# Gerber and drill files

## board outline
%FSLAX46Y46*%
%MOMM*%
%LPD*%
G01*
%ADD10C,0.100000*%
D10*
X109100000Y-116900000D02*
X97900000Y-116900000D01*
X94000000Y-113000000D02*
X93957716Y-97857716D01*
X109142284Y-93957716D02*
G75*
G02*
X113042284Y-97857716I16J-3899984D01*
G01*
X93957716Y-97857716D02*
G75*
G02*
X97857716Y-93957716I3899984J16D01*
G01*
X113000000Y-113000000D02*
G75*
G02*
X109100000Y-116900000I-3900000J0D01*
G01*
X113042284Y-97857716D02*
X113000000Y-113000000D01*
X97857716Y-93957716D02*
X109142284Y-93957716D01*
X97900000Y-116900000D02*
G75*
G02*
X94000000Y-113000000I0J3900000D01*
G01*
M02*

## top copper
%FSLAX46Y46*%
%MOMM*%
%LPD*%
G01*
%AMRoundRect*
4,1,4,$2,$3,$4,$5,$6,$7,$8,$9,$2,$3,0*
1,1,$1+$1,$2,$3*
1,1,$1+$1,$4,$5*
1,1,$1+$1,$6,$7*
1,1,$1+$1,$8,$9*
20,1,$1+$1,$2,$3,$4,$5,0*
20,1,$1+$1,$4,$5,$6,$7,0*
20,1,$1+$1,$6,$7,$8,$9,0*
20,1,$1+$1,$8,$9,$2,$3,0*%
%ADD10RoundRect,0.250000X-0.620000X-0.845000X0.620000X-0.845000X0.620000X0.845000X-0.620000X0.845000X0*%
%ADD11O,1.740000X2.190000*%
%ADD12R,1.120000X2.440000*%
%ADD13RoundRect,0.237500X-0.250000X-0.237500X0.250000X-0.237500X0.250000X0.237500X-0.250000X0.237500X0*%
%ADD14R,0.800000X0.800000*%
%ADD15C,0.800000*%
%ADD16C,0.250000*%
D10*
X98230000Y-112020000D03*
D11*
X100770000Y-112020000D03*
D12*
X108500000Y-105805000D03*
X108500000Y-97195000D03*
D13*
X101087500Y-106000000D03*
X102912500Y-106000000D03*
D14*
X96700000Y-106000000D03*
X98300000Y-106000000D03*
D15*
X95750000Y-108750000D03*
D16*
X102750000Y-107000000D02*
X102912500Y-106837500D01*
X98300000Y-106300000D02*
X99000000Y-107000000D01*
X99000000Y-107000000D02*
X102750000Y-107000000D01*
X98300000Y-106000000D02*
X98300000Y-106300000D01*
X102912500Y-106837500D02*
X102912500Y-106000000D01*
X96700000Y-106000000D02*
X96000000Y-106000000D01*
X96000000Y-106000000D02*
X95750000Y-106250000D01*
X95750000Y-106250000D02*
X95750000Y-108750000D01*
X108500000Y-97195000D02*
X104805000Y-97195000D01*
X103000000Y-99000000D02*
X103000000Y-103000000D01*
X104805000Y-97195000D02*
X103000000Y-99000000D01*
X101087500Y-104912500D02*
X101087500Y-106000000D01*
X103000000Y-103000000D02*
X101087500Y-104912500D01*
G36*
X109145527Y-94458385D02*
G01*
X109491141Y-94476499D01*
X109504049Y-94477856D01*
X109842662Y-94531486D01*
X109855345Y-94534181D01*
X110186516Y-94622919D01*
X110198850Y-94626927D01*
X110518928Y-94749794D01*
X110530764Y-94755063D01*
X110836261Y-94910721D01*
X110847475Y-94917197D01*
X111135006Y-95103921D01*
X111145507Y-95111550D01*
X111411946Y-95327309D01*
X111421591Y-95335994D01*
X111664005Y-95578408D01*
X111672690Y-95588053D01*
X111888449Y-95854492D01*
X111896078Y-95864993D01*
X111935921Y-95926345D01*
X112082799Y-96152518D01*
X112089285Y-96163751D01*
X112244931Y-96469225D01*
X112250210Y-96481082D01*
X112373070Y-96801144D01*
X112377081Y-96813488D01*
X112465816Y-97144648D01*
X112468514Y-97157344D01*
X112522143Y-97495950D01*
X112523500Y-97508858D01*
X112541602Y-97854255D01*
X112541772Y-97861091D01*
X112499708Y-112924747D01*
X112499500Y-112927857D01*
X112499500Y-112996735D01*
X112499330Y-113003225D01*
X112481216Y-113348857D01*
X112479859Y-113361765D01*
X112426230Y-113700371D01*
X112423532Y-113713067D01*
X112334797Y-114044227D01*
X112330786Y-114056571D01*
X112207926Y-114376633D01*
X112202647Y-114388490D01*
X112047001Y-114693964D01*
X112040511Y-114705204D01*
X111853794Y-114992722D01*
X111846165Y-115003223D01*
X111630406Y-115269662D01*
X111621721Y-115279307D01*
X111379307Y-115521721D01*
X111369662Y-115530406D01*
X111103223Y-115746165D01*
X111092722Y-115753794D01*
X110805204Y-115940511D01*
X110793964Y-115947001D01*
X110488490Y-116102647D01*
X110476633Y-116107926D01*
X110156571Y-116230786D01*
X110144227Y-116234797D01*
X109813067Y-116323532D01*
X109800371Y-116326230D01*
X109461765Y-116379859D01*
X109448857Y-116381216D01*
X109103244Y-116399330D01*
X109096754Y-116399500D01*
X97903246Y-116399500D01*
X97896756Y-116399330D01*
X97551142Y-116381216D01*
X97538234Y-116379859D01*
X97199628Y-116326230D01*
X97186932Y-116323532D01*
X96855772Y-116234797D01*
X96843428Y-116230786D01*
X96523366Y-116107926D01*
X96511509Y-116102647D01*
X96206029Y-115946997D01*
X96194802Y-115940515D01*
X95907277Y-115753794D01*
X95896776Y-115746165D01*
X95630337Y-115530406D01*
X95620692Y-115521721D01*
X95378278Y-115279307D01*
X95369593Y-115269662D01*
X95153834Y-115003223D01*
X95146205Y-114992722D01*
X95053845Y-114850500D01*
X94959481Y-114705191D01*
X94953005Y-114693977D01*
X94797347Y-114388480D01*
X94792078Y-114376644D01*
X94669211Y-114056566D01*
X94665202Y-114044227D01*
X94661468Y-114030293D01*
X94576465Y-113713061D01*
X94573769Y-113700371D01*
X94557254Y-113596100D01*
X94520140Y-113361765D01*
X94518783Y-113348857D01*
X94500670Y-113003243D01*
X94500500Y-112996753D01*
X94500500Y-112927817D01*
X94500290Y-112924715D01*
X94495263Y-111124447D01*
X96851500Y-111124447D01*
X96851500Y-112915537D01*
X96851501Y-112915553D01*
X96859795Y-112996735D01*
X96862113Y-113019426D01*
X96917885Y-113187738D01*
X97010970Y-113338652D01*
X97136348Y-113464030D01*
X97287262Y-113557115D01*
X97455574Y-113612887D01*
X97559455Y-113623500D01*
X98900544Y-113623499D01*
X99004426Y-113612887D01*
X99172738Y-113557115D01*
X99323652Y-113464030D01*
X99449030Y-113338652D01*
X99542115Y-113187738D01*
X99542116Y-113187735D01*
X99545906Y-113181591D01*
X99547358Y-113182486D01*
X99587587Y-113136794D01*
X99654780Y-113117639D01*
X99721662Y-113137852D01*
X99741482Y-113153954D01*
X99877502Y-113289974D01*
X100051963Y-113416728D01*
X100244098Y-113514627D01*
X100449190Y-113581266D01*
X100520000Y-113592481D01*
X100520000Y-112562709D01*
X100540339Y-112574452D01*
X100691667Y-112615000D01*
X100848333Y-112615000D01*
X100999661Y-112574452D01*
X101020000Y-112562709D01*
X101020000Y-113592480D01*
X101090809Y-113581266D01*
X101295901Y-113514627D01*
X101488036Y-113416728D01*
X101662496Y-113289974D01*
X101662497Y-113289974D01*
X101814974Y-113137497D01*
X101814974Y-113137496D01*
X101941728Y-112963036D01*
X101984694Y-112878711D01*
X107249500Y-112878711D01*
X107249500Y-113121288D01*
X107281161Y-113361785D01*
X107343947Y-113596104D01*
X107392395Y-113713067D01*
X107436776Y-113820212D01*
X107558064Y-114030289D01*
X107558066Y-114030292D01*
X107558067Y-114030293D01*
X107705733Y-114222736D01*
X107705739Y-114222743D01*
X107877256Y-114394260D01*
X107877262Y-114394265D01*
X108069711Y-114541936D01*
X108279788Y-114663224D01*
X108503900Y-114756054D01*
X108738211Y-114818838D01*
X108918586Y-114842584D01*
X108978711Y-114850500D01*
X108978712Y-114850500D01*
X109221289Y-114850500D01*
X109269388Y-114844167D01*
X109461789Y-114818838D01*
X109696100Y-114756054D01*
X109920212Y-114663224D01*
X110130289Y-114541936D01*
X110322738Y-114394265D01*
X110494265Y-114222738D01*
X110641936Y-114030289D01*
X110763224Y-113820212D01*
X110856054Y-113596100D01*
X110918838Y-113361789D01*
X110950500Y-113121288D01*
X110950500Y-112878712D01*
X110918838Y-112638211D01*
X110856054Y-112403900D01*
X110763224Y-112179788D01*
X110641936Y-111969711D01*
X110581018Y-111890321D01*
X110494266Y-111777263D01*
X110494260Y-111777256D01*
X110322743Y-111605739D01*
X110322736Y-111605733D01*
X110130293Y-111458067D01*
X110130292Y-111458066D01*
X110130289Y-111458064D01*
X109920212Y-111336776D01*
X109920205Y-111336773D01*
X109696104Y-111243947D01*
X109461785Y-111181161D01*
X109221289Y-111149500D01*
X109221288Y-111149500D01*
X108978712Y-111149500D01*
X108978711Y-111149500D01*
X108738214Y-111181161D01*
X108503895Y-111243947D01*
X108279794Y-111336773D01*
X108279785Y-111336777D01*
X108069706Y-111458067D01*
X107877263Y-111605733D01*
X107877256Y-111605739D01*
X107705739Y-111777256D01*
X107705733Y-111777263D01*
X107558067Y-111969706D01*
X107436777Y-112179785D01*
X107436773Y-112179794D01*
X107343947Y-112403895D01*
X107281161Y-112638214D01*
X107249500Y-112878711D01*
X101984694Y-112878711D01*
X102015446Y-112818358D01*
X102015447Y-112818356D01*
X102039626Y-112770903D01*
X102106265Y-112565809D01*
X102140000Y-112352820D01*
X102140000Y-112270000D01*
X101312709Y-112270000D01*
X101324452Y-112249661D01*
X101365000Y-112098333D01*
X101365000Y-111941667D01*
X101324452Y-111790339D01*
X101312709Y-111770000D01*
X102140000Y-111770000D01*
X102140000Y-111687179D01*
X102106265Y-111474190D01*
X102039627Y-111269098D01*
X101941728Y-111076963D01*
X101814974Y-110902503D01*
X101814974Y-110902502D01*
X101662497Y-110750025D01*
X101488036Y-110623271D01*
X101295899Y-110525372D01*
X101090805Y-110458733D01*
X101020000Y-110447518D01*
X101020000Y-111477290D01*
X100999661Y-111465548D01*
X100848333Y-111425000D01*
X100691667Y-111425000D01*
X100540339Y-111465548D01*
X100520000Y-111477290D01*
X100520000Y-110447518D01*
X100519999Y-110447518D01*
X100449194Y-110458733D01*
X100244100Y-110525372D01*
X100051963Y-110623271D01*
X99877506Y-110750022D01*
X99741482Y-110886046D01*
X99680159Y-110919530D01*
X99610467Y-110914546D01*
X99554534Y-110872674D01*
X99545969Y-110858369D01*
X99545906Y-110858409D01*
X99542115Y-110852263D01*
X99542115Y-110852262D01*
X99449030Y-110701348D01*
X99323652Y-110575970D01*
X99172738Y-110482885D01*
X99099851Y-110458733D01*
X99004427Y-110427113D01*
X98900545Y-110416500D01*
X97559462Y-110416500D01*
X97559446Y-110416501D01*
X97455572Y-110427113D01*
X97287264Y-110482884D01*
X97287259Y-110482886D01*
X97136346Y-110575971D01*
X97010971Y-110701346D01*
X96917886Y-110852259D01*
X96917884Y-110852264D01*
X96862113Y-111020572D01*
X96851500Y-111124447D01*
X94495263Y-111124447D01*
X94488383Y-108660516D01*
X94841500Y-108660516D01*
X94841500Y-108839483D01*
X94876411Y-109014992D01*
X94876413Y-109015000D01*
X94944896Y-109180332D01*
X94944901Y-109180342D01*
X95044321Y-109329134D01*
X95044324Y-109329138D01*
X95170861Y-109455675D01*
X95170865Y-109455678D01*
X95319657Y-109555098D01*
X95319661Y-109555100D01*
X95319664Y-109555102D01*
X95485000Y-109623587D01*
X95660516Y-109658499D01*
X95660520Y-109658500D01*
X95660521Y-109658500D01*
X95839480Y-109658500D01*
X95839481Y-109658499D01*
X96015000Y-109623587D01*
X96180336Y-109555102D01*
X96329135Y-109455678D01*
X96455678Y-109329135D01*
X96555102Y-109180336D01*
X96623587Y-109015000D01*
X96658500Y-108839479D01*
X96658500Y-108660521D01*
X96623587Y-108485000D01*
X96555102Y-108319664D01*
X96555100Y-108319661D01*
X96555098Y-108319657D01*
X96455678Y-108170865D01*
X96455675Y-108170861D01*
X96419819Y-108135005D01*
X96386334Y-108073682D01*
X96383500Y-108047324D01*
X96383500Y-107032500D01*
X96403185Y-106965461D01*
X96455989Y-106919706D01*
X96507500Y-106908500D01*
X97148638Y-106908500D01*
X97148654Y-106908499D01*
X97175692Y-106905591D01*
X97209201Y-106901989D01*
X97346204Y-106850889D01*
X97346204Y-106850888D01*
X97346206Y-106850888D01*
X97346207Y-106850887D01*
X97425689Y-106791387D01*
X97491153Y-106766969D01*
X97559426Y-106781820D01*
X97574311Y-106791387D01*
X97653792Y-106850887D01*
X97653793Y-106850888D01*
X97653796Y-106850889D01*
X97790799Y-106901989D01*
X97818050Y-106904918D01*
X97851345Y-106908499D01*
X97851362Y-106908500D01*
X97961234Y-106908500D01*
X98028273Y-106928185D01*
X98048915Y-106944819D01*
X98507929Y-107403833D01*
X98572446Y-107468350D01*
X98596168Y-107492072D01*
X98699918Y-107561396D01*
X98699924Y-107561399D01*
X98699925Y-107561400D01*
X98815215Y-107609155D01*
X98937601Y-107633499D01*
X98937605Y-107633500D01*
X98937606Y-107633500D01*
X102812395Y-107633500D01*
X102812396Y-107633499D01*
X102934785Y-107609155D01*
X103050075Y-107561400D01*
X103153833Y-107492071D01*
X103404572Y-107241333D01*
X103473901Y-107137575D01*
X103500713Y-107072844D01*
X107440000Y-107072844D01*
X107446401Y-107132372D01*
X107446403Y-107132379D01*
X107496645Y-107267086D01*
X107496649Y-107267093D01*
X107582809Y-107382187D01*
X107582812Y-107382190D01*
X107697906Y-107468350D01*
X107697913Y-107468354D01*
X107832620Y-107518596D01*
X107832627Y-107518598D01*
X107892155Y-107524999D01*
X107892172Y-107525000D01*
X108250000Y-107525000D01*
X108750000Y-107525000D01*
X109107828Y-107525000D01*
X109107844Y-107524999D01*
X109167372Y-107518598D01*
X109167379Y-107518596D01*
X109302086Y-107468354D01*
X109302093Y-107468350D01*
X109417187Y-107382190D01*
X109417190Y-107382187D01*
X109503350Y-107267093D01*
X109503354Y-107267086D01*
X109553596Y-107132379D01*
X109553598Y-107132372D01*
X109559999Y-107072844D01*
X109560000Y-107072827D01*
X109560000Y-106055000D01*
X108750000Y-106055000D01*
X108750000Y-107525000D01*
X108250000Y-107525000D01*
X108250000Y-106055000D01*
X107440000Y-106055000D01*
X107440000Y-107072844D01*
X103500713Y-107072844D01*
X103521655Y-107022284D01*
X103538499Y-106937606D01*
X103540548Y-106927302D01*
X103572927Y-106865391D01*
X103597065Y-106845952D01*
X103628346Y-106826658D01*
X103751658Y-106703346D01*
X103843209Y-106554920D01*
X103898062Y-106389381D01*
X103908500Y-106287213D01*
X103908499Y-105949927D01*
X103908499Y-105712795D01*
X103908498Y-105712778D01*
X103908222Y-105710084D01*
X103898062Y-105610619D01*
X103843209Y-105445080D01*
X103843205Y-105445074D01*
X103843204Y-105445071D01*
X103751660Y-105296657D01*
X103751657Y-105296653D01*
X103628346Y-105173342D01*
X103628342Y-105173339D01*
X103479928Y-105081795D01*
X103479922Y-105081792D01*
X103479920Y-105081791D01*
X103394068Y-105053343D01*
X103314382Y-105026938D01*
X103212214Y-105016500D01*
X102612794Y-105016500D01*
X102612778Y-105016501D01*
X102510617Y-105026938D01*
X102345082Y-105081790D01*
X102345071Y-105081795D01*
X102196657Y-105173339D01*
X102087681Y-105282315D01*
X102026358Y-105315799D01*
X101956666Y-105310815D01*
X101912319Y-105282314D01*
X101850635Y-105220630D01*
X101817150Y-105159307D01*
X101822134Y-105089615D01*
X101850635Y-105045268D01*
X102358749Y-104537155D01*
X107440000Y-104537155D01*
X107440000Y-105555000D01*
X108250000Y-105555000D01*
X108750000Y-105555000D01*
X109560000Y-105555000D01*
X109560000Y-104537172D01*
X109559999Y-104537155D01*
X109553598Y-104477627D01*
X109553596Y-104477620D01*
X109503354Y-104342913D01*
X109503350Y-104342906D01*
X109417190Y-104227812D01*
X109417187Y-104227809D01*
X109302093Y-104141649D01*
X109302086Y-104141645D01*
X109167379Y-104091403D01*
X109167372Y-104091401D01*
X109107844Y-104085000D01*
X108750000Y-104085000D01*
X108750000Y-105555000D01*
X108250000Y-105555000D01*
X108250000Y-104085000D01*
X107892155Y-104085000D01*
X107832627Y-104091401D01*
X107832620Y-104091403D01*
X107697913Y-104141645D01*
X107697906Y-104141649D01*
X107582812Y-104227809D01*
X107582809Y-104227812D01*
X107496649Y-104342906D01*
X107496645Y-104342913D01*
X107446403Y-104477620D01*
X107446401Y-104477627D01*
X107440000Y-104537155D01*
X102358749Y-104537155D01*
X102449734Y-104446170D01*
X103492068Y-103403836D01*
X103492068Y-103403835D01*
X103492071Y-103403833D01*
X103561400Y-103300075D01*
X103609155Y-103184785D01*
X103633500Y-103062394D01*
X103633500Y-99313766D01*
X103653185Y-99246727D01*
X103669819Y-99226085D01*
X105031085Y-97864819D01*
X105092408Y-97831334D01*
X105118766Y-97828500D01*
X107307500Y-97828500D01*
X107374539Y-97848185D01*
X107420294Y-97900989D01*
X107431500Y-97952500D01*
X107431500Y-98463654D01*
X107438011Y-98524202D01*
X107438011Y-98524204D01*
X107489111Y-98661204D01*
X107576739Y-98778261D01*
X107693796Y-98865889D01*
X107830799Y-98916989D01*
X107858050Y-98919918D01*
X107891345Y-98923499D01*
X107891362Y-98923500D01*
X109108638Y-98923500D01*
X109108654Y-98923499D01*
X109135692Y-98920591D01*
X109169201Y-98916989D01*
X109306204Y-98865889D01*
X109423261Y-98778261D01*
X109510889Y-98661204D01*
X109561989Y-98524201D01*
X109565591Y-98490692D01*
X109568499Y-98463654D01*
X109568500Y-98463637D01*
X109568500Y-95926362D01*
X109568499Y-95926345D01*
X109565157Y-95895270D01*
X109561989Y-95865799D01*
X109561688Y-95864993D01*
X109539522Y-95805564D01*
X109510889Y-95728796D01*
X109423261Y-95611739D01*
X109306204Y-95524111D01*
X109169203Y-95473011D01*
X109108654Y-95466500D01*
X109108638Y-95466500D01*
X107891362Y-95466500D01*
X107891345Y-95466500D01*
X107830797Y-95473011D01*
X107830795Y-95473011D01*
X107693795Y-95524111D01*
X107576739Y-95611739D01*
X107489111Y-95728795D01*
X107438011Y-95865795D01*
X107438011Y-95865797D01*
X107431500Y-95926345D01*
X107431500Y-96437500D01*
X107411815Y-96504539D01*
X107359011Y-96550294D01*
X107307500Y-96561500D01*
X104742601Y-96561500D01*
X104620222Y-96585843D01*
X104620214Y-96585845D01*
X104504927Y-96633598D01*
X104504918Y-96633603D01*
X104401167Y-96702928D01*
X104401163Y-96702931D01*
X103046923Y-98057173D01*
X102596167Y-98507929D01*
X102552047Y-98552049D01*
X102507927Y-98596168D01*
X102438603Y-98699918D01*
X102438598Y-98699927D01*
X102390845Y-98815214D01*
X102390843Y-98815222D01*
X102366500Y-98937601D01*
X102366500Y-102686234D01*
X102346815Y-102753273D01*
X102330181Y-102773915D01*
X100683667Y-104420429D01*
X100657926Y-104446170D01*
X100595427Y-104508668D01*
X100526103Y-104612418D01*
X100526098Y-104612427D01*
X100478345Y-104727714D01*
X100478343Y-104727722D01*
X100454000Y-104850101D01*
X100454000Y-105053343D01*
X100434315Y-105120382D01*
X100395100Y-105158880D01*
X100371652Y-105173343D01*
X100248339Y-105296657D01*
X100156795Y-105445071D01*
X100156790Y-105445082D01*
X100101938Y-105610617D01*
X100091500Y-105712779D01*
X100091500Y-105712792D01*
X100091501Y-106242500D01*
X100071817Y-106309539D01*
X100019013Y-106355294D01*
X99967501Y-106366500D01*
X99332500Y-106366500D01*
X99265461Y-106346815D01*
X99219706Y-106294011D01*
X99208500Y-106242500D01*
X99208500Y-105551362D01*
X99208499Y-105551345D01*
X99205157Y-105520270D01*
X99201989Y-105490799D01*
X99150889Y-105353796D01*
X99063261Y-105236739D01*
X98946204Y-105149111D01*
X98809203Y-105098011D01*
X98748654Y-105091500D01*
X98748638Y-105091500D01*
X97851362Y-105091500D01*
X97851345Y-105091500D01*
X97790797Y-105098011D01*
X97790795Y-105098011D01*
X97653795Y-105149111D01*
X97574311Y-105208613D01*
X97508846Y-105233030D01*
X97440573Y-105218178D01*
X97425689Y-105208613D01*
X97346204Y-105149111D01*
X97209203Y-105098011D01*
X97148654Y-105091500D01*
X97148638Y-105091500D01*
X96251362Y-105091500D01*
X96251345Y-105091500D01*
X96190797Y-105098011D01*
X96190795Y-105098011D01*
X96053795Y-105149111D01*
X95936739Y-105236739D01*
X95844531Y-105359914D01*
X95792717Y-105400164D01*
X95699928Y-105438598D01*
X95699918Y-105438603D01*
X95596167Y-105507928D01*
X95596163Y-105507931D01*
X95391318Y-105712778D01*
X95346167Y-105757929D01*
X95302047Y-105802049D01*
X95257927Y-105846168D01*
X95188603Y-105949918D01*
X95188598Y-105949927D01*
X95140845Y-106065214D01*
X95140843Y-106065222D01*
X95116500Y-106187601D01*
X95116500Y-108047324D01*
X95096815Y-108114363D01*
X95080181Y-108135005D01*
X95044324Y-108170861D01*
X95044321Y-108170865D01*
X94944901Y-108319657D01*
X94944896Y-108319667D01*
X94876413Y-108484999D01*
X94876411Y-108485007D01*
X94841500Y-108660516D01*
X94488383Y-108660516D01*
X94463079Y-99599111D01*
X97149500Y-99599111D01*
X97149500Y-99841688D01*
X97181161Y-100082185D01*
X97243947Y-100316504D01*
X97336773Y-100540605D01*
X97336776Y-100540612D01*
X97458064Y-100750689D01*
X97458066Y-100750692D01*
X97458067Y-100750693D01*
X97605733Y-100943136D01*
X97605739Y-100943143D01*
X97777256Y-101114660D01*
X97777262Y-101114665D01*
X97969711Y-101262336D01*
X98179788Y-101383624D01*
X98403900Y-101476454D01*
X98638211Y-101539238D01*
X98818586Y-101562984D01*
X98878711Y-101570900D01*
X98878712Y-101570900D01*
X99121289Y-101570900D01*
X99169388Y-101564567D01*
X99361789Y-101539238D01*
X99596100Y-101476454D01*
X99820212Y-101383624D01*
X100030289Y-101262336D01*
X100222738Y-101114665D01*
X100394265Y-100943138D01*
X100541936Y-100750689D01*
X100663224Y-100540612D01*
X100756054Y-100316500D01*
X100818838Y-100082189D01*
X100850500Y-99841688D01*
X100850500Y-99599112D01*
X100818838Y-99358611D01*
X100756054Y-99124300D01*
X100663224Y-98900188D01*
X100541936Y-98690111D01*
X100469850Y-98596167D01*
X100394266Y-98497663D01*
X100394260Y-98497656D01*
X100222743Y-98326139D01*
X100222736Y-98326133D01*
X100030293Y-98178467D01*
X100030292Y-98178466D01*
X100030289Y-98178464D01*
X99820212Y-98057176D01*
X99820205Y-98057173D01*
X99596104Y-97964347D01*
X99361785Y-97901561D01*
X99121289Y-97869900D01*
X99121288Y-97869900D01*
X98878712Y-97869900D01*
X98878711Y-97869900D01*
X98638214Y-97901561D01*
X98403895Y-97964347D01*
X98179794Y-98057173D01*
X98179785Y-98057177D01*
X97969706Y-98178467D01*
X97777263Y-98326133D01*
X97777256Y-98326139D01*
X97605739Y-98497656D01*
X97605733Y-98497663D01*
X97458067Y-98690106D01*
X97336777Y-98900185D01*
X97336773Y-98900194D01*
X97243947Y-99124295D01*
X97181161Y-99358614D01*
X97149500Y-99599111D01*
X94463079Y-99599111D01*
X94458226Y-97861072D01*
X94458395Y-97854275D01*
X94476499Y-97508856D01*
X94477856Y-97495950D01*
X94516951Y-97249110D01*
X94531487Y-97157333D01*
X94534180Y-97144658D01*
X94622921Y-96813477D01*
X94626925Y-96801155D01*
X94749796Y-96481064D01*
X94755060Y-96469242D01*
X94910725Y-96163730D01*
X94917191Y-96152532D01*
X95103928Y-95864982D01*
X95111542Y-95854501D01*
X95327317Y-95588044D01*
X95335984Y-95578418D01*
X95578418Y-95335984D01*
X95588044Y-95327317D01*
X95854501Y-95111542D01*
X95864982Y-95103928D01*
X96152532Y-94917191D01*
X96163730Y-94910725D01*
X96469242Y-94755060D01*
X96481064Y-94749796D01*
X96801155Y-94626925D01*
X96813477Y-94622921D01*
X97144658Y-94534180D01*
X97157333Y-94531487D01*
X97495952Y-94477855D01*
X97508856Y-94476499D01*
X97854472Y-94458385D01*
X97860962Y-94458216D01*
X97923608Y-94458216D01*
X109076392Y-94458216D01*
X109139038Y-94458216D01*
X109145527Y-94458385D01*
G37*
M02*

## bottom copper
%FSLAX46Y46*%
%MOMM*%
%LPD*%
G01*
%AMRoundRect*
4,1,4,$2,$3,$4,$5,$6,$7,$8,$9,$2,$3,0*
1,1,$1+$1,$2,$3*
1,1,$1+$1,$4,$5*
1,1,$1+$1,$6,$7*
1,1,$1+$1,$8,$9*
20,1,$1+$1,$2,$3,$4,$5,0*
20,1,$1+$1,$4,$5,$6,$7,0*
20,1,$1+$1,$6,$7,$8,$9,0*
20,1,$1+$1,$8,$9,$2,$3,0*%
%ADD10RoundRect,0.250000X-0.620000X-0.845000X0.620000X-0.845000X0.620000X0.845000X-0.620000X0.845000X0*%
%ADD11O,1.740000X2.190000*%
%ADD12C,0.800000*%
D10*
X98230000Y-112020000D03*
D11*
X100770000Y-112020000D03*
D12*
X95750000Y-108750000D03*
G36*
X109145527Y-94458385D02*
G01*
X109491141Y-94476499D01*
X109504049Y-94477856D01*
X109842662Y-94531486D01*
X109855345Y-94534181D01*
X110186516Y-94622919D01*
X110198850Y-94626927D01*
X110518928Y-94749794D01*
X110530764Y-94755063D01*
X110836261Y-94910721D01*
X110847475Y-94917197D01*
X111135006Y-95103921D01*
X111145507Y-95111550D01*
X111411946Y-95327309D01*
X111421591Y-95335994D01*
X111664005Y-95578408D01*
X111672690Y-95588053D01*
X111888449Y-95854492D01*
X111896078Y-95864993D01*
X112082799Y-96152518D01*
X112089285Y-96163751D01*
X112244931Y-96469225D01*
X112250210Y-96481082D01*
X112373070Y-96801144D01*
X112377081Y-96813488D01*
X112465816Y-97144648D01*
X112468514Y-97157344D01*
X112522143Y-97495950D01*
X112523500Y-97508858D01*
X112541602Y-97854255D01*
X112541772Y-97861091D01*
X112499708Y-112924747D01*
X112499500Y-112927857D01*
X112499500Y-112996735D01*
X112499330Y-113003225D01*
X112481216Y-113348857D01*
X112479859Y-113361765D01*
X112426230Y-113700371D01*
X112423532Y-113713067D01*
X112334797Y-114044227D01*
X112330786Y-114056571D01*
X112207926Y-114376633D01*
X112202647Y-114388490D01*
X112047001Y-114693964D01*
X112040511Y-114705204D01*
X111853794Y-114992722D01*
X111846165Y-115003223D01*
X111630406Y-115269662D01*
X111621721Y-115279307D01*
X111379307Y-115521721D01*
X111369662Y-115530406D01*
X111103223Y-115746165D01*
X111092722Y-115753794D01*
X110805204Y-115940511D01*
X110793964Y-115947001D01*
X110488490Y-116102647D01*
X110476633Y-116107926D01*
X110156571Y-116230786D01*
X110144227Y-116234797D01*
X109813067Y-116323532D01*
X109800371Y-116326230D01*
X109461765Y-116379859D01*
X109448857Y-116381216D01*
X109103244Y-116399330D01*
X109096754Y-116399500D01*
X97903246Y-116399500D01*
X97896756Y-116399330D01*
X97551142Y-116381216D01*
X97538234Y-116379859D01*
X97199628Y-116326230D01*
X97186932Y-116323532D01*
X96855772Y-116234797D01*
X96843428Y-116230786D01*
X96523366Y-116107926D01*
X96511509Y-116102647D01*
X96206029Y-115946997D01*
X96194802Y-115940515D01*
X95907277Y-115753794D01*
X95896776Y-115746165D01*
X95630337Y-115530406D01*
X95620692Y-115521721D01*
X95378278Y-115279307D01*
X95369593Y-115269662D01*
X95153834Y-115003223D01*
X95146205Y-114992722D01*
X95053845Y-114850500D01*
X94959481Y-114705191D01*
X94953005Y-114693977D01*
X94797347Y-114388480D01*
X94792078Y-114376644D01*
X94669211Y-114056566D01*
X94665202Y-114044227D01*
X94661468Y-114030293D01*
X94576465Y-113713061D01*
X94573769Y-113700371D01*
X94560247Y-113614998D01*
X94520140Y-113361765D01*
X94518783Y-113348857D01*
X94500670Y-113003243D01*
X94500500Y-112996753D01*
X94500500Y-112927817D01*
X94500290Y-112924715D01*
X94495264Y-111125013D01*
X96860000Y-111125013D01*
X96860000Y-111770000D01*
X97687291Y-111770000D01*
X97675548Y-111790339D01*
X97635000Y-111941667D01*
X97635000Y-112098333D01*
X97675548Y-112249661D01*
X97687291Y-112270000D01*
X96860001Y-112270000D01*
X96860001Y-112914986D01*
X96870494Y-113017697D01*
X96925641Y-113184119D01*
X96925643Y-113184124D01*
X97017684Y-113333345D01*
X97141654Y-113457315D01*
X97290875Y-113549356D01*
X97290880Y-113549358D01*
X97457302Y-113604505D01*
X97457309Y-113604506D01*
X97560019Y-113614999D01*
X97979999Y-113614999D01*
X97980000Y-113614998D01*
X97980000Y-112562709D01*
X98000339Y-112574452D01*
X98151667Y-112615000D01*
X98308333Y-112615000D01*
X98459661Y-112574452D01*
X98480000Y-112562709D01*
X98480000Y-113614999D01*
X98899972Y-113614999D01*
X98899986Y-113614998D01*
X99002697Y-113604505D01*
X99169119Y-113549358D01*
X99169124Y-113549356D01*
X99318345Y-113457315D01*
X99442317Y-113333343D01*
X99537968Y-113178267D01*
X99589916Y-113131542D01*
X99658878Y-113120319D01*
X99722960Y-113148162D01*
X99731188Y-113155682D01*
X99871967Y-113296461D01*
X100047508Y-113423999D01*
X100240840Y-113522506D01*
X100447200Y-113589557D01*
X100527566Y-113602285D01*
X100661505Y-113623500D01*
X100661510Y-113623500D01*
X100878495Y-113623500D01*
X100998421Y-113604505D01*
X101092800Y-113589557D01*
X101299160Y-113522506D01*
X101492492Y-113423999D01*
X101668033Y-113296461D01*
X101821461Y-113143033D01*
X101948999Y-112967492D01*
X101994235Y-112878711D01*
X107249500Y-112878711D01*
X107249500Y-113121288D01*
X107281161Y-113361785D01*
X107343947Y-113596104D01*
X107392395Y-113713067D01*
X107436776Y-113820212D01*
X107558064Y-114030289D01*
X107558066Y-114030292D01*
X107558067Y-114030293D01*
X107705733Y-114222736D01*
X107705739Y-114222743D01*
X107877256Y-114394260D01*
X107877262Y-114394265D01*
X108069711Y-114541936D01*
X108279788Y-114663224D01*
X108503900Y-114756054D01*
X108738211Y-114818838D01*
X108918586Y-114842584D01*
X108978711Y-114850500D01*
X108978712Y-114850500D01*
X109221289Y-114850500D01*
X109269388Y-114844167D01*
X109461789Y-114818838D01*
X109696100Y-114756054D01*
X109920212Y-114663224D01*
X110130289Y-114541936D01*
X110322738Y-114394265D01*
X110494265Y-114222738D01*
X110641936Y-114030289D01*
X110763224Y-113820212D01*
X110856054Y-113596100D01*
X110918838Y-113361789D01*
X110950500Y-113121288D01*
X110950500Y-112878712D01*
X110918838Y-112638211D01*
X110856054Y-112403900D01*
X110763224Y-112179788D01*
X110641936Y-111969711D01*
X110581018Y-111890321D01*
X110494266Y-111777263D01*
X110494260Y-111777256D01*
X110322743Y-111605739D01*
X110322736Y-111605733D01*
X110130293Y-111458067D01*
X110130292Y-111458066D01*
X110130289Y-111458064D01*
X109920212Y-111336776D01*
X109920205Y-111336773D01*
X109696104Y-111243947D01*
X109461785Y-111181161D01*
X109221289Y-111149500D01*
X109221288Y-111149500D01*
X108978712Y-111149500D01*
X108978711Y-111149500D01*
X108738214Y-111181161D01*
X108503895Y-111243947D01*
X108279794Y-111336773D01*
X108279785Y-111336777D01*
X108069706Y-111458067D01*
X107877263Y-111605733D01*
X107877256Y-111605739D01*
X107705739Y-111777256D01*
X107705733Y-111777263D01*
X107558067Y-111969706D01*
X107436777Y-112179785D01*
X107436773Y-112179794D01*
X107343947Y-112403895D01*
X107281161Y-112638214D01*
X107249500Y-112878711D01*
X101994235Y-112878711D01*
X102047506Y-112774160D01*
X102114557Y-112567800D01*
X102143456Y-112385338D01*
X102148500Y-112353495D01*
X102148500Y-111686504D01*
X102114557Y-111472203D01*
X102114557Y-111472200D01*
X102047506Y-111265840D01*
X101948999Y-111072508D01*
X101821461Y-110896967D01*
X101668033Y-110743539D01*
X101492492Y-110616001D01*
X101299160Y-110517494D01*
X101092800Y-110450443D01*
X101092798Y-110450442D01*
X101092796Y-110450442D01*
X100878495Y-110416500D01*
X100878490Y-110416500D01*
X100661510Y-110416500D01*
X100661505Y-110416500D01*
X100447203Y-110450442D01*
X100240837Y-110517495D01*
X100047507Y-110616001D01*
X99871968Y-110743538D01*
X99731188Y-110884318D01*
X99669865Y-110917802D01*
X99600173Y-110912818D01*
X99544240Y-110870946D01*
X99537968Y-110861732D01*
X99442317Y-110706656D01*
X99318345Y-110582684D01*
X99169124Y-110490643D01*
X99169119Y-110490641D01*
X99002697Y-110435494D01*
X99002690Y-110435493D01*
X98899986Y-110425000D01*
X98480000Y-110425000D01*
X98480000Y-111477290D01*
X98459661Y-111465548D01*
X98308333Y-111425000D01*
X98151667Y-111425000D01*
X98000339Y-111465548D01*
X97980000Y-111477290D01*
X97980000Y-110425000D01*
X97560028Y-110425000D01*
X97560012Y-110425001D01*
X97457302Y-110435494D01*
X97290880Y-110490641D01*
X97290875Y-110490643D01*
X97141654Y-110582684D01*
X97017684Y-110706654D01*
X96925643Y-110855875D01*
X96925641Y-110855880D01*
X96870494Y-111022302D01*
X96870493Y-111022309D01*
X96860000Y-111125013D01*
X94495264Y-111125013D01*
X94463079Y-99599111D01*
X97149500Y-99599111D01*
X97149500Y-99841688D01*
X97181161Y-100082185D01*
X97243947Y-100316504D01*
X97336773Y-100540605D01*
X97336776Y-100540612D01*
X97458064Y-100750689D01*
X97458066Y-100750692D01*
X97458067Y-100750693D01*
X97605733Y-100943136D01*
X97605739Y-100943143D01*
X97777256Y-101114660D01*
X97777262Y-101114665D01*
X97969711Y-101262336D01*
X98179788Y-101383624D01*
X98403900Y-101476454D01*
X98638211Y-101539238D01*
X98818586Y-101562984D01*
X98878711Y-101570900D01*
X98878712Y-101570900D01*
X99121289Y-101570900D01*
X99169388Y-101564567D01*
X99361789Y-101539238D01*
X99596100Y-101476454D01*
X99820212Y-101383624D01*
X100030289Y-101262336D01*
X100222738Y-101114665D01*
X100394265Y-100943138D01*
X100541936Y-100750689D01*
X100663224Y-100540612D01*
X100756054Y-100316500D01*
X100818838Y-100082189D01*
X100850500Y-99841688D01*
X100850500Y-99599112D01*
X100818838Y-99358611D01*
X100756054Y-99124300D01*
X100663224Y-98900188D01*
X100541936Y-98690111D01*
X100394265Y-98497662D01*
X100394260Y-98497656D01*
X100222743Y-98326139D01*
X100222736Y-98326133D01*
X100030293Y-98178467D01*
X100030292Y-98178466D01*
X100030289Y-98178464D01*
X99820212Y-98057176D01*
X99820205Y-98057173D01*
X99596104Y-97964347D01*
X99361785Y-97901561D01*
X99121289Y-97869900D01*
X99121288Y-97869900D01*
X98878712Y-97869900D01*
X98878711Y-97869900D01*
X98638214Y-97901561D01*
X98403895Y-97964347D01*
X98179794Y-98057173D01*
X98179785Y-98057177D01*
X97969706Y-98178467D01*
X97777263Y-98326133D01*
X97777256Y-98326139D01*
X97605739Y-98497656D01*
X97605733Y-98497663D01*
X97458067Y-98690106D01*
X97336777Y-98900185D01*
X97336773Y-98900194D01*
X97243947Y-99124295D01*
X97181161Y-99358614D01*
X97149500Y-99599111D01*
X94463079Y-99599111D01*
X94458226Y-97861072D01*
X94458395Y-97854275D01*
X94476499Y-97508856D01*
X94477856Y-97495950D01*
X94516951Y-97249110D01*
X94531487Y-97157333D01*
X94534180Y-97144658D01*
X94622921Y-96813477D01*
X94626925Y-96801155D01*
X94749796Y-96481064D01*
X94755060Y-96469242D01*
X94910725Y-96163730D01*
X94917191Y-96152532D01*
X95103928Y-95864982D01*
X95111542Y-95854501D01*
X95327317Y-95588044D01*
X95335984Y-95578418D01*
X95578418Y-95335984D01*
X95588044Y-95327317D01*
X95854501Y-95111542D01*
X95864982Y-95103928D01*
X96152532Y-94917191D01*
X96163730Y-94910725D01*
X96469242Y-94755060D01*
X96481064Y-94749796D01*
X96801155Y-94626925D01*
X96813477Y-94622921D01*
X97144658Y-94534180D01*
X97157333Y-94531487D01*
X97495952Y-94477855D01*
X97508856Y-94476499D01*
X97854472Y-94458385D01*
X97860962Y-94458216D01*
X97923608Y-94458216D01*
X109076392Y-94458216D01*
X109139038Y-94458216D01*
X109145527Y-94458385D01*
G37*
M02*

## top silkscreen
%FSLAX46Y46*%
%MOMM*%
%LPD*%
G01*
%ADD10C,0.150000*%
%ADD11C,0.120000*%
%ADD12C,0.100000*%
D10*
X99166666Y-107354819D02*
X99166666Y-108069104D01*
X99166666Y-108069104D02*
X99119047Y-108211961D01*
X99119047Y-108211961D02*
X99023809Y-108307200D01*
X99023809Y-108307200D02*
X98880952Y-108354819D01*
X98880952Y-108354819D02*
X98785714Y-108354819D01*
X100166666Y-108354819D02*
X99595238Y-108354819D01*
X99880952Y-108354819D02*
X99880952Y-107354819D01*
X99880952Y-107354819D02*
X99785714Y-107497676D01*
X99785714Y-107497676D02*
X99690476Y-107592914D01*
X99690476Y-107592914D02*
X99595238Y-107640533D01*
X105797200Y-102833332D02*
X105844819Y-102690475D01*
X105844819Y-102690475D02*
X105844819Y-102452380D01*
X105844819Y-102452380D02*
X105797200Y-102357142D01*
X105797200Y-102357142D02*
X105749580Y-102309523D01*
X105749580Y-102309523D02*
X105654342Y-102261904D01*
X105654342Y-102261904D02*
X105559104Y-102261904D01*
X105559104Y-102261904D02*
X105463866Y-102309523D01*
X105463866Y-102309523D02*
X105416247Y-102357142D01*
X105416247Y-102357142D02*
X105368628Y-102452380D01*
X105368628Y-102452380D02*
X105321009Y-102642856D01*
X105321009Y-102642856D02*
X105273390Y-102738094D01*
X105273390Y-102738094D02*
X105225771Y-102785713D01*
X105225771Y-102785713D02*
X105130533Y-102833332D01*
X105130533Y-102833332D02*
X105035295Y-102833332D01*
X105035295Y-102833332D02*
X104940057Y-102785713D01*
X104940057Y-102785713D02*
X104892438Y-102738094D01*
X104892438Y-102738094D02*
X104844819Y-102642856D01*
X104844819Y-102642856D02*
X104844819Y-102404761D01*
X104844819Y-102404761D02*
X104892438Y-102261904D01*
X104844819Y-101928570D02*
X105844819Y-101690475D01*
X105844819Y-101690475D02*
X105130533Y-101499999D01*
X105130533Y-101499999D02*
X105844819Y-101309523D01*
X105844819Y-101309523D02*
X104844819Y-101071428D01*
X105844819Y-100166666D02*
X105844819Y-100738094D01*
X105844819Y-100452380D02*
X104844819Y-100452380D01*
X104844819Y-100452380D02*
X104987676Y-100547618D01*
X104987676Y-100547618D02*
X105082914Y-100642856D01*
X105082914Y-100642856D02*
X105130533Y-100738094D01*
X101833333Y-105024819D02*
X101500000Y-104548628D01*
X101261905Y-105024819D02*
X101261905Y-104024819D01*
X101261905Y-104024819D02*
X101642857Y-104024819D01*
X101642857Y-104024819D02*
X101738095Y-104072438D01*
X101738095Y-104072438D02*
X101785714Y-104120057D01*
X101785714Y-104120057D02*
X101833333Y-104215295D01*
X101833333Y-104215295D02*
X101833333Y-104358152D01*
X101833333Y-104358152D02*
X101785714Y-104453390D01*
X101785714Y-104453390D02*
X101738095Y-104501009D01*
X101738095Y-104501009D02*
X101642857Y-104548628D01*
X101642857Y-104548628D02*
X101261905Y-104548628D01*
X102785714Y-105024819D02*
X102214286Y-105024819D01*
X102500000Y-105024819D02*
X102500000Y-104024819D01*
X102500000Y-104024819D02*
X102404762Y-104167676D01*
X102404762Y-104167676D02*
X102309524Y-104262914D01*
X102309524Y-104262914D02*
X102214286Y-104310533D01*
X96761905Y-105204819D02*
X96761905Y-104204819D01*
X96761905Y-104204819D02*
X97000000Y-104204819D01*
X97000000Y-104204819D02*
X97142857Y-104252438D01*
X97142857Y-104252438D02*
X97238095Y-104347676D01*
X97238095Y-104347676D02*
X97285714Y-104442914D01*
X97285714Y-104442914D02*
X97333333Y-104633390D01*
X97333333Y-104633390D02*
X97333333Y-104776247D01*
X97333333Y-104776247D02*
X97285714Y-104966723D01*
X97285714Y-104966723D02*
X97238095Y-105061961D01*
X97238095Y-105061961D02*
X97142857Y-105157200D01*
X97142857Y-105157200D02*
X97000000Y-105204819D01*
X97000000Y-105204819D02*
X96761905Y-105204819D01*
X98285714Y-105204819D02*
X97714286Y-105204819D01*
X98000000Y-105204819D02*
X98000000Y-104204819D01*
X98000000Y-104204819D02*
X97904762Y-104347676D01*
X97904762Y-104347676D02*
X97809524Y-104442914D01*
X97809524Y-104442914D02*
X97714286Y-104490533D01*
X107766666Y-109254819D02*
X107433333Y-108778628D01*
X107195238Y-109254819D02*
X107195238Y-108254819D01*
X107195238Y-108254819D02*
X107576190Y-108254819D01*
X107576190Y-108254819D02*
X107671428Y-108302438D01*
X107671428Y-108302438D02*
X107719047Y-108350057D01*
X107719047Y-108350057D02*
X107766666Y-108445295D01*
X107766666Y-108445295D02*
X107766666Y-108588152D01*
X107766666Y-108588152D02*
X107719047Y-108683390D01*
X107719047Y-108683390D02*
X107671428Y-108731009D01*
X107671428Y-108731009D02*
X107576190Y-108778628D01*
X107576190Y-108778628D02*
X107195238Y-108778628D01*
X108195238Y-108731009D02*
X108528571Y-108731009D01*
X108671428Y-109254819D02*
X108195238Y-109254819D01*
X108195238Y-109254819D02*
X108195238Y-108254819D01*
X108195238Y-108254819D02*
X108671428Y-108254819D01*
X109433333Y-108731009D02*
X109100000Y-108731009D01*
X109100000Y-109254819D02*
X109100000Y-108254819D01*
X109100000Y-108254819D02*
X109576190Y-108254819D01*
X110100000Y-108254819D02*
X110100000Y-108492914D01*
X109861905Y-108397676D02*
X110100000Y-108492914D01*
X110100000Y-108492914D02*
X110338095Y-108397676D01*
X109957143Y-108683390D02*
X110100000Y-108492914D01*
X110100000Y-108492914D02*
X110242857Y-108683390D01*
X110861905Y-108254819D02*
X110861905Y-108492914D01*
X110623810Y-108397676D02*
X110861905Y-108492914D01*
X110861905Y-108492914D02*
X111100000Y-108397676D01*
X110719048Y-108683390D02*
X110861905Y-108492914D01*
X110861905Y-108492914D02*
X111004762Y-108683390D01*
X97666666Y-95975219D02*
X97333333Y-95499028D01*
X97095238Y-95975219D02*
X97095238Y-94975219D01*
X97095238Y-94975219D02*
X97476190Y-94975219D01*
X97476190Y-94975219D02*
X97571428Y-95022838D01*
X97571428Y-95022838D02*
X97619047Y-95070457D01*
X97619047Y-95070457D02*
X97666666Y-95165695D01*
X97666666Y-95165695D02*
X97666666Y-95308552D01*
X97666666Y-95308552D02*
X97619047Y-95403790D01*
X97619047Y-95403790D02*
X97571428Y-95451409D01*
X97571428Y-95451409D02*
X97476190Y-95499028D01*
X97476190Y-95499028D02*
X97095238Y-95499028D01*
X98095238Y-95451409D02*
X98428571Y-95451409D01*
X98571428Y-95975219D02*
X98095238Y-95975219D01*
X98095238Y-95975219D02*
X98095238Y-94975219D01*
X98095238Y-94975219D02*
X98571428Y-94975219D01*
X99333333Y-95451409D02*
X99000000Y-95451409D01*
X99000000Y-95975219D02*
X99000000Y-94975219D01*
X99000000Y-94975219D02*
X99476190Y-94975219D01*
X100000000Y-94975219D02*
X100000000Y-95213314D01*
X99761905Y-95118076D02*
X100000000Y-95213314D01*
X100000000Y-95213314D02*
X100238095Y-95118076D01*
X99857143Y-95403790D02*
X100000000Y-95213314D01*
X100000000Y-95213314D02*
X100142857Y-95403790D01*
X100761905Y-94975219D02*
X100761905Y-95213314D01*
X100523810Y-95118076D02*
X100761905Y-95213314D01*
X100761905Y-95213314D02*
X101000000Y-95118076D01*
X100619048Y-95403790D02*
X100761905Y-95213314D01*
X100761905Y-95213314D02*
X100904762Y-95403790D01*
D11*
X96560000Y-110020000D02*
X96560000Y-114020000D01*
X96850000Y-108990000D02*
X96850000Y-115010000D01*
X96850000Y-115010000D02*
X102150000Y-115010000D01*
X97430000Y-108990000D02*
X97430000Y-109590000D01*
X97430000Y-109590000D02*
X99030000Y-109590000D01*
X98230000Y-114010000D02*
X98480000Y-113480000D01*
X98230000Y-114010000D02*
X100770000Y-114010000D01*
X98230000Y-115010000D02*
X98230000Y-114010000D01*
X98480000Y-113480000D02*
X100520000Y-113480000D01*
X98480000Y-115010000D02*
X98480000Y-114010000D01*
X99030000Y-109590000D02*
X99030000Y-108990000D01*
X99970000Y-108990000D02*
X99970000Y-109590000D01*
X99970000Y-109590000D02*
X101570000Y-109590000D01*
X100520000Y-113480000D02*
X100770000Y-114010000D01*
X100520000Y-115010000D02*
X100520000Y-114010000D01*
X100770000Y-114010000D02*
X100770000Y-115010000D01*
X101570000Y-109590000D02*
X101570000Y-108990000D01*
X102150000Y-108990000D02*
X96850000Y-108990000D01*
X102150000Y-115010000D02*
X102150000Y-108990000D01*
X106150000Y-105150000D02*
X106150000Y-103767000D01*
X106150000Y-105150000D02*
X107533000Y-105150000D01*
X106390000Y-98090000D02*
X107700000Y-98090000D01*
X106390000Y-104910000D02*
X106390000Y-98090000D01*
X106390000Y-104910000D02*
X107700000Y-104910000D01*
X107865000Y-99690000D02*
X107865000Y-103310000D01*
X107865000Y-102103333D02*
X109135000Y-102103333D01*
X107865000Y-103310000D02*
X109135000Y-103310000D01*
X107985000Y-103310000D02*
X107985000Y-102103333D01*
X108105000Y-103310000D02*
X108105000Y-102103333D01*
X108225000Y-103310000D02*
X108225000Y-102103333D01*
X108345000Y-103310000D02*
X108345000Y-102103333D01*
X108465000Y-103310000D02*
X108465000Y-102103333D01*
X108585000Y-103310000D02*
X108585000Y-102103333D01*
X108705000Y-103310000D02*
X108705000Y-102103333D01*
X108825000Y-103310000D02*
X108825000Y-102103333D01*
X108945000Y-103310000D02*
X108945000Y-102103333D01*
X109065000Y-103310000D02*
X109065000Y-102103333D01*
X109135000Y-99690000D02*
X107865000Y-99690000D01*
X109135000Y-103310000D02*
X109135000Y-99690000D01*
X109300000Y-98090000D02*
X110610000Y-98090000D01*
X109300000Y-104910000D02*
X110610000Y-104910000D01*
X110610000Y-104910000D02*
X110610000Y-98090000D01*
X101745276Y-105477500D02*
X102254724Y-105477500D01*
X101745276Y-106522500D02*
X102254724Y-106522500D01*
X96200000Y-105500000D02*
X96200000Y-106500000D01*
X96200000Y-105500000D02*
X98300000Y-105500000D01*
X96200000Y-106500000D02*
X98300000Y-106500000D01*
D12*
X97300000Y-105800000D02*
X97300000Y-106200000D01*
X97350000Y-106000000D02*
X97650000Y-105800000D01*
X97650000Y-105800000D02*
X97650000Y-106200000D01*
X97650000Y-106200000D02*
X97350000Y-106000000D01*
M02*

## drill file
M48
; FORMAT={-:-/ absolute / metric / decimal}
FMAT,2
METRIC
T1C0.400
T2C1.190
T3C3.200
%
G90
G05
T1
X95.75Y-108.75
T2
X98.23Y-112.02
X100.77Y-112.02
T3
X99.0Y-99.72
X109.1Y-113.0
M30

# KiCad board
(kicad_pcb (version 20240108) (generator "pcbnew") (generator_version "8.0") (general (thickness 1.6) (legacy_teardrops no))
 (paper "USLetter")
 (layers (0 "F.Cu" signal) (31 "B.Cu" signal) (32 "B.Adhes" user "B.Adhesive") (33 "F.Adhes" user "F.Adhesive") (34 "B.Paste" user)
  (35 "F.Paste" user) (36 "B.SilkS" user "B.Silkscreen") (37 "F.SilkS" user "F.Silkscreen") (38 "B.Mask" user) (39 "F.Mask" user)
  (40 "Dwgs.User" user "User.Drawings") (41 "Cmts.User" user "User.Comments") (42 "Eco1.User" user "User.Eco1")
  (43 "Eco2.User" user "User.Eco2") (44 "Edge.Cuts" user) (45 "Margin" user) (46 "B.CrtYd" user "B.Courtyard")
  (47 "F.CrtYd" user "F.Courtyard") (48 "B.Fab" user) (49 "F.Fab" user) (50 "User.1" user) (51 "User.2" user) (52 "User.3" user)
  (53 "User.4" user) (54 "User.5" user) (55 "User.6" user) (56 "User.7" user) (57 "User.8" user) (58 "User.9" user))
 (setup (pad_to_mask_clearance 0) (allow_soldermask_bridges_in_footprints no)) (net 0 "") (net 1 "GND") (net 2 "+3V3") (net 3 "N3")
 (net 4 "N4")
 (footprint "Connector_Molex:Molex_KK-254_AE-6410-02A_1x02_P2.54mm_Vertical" (layer "F.Cu") (at 98.23 112.02)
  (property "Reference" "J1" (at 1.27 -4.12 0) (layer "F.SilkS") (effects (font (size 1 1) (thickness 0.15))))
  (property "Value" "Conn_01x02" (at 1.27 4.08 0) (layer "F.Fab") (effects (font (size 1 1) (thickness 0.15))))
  (fp_line (start -1.67 -2) (end -1.67 2) (stroke (width 0.12) (type solid)) (layer "F.SilkS"))
  (fp_line (start -1.38 -3.03) (end -1.38 2.99) (stroke (width 0.12) (type solid)) (layer "F.SilkS"))
  (fp_line (start -1.38 2.99) (end 3.92 2.99) (stroke (width 0.12) (type solid)) (layer "F.SilkS"))
  (fp_line (start -0.8 -3.03) (end -0.8 -2.43) (stroke (width 0.12) (type solid)) (layer "F.SilkS"))
  (fp_line (start -0.8 -2.43) (end 0.8 -2.43) (stroke (width 0.12) (type solid)) (layer "F.SilkS"))
  (fp_line (start 0 1.99) (end 0.25 1.46) (stroke (width 0.12) (type solid)) (layer "F.SilkS"))
  (fp_line (start 0 1.99) (end 2.54 1.99) (stroke (width 0.12) (type solid)) (layer "F.SilkS"))
  (fp_line (start 0 2.99) (end 0 1.99) (stroke (width 0.12) (type solid)) (layer "F.SilkS"))
  (fp_line (start 0.25 1.46) (end 2.29 1.46) (stroke (width 0.12) (type solid)) (layer "F.SilkS"))
  (fp_line (start 0.25 2.99) (end 0.25 1.99) (stroke (width 0.12) (type solid)) (layer "F.SilkS"))
  (fp_line (start 0.8 -2.43) (end 0.8 -3.03) (stroke (width 0.12) (type solid)) (layer "F.SilkS"))
  (fp_line (start 1.74 -3.03) (end 1.74 -2.43) (stroke (width 0.12) (type solid)) (layer "F.SilkS"))
  (fp_line (start 1.74 -2.43) (end 3.34 -2.43) (stroke (width 0.12) (type solid)) (layer "F.SilkS"))
  (fp_line (start 2.29 1.46) (end 2.54 1.99) (stroke (width 0.12) (type solid)) (layer "F.SilkS"))
  (fp_line (start 2.29 2.99) (end 2.29 1.99) (stroke (width 0.12) (type solid)) (layer "F.SilkS"))
  (fp_line (start 2.54 1.99) (end 2.54 2.99) (stroke (width 0.12) (type solid)) (layer "F.SilkS"))
  (fp_line (start 3.34 -2.43) (end 3.34 -3.03) (stroke (width 0.12) (type solid)) (layer "F.SilkS"))
  (fp_line (start 3.92 -3.03) (end -1.38 -3.03) (stroke (width 0.12) (type solid)) (layer "F.SilkS"))
  (fp_line (start 3.92 2.99) (end 3.92 -3.03) (stroke (width 0.12) (type solid)) (layer "F.SilkS"))
  (pad "1" thru_hole roundrect (at 0 0) (size 1.74 2.19) (drill 1.19) (layers "*.Cu" "*.Mask") (remove_unused_layers no)
   (roundrect_rratio 0.143678) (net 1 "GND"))
  (pad "2" thru_hole oval (at 2.54 0) (size 1.74 2.19) (drill 1.19) (layers "*.Cu" "*.Mask") (remove_unused_layers no) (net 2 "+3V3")))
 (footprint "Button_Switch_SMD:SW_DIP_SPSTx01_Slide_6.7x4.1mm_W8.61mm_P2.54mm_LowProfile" (layer "F.Cu") (at 108.5 101.5 90)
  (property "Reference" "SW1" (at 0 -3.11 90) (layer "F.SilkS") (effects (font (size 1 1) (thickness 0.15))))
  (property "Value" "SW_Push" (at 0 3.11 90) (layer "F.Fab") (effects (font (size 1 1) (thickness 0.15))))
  (fp_line (start -3.65 -2.35) (end -2.267 -2.35) (stroke (width 0.12) (type solid)) (layer "F.SilkS"))
  (fp_line (start -3.65 -2.35) (end -3.65 -0.967) (stroke (width 0.12) (type solid)) (layer "F.SilkS"))
  (fp_line (start 3.41 -2.11) (end 3.41 -0.8) (stroke (width 0.12) (type solid)) (layer "F.SilkS"))
  (fp_line (start -3.41 -2.11) (end 3.41 -2.11) (stroke (width 0.12) (type solid)) (layer "F.SilkS"))
  (fp_line (start -3.41 -2.11) (end -3.41 -0.8) (stroke (width 0.12) (type solid)) (layer "F.SilkS"))
  (fp_line (start 1.81 -0.635) (end -1.81 -0.635) (stroke (width 0.12) (type solid)) (layer "F.SilkS"))
  (fp_line (start -0.603333 -0.635) (end -0.603333 0.635) (stroke (width 0.12) (type solid)) (layer "F.SilkS"))
  (fp_line (start -1.81 -0.635) (end -1.81 0.635) (stroke (width 0.12) (type solid)) (layer "F.SilkS"))
  (fp_line (start -1.81 -0.515) (end -0.603333 -0.515) (stroke (width 0.12) (type solid)) (layer "F.SilkS"))
  (fp_line (start -1.81 -0.395) (end -0.603333 -0.395) (stroke (width 0.12) (type solid)) (layer "F.SilkS"))
  (fp_line (start -1.81 -0.275) (end -0.603333 -0.275) (stroke (width 0.12) (type solid)) (layer "F.SilkS"))
  (fp_line (start -1.81 -0.155) (end -0.603333 -0.155) (stroke (width 0.12) (type solid)) (layer "F.SilkS"))
  (fp_line (start -1.81 -0.035) (end -0.603333 -0.035) (stroke (width 0.12) (type solid)) (layer "F.SilkS"))
  (fp_line (start -1.81 0.085) (end -0.603333 0.085) (stroke (width 0.12) (type solid)) (layer "F.SilkS"))
  (fp_line (start -1.81 0.205) (end -0.603333 0.205) (stroke (width 0.12) (type solid)) (layer "F.SilkS"))
  (fp_line (start -1.81 0.325) (end -0.603333 0.325) (stroke (width 0.12) (type solid)) (layer "F.SilkS"))
  (fp_line (start -1.81 0.445) (end -0.603333 0.445) (stroke (width 0.12) (type solid)) (layer "F.SilkS"))
  (fp_line (start -1.81 0.565) (end -0.603333 0.565) (stroke (width 0.12) (type solid)) (layer "F.SilkS"))
  (fp_line (start 1.81 0.635) (end 1.81 -0.635) (stroke (width 0.12) (type solid)) (layer "F.SilkS"))
  (fp_line (start -1.81 0.635) (end 1.81 0.635) (stroke (width 0.12) (type solid)) (layer "F.SilkS"))
  (fp_line (start 3.41 0.8) (end 3.41 2.11) (stroke (width 0.12) (type solid)) (layer "F.SilkS"))
  (fp_line (start -3.41 0.8) (end -3.41 2.11) (stroke (width 0.12) (type solid)) (layer "F.SilkS"))
  (fp_line (start -3.41 2.11) (end 3.41 2.11) (stroke (width 0.12) (type solid)) (layer "F.SilkS"))
  (pad "1" smd rect (at -4.305 0 90) (size 2.44 1.12) (layers "F.Cu" "F.Paste" "F.Mask") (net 2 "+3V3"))
  (pad "2" smd rect (at 4.305 0 90) (size 2.44 1.12) (layers "F.Cu" "F.Paste" "F.Mask") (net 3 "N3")))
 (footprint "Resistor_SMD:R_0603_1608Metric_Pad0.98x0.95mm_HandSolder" (layer "F.Cu") (at 102 106)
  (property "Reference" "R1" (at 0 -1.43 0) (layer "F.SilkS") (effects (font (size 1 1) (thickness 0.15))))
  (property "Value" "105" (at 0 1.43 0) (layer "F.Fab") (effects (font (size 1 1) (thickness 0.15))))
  (fp_line (start -0.254724 -0.5225) (end 0.254724 -0.5225) (stroke (width 0.12) (type solid)) (layer "F.SilkS"))
  (fp_line (start -0.254724 0.5225) (end 0.254724 0.5225) (stroke (width 0.12) (type solid)) (layer "F.SilkS"))
  (pad "1" smd roundrect (at -0.9125 0) (size 0.975 0.95) (layers "F.Cu" "F.Paste" "F.Mask") (roundrect_rratio 0.25) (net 3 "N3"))
  (pad "2" smd roundrect (at 0.9125 0) (size 0.975 0.95) (layers "F.Cu" "F.Paste" "F.Mask") (roundrect_rratio 0.25) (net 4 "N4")))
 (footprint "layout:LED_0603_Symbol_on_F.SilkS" (layer "F.Cu") (at 97.5 106)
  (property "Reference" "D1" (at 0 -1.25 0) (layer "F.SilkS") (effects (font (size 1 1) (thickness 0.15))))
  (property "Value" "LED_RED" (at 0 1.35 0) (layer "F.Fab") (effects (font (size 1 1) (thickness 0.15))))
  (fp_line (start -1.3 -0.5) (end -1.3 0.5) (stroke (width 0.12) (type solid)) (layer "F.SilkS"))
  (fp_line (start -1.3 -0.5) (end 0.8 -0.5) (stroke (width 0.12) (type solid)) (layer "F.SilkS"))
  (fp_line (start -1.3 0.5) (end 0.8 0.5) (stroke (width 0.12) (type solid)) (layer "F.SilkS"))
  (fp_line (start -0.2 -0.2) (end -0.2 0.2) (stroke (width 0.1) (type solid)) (layer "F.SilkS"))
  (fp_line (start -0.15 0) (end 0.15 -0.2) (stroke (width 0.1) (type solid)) (layer "F.SilkS"))
  (fp_line (start 0.15 -0.2) (end 0.15 0.2) (stroke (width 0.1) (type solid)) (layer "F.SilkS"))
  (fp_line (start 0.15 0.2) (end -0.15 0) (stroke (width 0.1) (type solid)) (layer "F.SilkS"))
  (pad "1" smd rect (at -0.8 0 180) (size 0.8 0.8) (layers "F.Cu" "F.Paste" "F.Mask") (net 1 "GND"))
  (pad "2" smd rect (at 0.8 0 180) (size 0.8 0.8) (layers "F.Cu" "F.Paste" "F.Mask") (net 4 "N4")))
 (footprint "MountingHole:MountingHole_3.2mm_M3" (layer "F.Cu") (at 109.1 113)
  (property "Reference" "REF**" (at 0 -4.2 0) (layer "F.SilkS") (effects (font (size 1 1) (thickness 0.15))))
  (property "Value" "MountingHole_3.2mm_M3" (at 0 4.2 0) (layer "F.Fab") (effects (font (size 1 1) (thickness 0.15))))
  (pad "" np_thru_hole circle (at 0 0) (size 3.2 3.2) (drill 3.2) (layers "*.Cu" "*.Mask")))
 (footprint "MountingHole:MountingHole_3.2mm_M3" (layer "F.Cu") (at 99 99.7204)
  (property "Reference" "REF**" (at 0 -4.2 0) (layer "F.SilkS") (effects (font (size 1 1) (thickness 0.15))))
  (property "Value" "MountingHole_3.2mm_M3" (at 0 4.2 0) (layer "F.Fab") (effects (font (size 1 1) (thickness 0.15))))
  (pad "" np_thru_hole circle (at 0 0) (size 3.2 3.2) (drill 3.2) (layers "*.Cu" "*.Mask")))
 (gr_line (start 109.1 116.9) (end 97.9 116.9) (stroke (width 0.1) (type default)) (layer "Edge.Cuts"))
 (gr_line (start 94 113) (end 93.957716 97.857716) (stroke (width 0.1) (type default)) (layer "Edge.Cuts"))
 (gr_arc (start 109.142284 93.957716) (mid 111.9 95.1) (end 113.042284 97.857716) (stroke (width 0.1) (type default)) (layer "Edge.Cuts"))
 (gr_arc (start 93.957716 97.857716) (mid 95.1 95.1) (end 97.857716 93.957716) (stroke (width 0.1) (type default)) (layer "Edge.Cuts"))
 (gr_arc (start 113 113) (mid 111.857716 115.757716) (end 109.1 116.9) (stroke (width 0.1) (type default)) (layer "Edge.Cuts"))
 (gr_line (start 113.042284 97.857716) (end 113 113) (stroke (width 0.1) (type default)) (layer "Edge.Cuts"))
 (gr_line (start 97.857716 93.957716) (end 109.142284 93.957716) (stroke (width 0.1) (type default)) (layer "Edge.Cuts"))
 (gr_arc (start 97.9 116.9) (mid 95.142284 115.757716) (end 94 113) (stroke (width 0.1) (type default)) (layer "Edge.Cuts"))
 (segment (start 102.75 107) (end 102.9125 106.8375) (width 0.25) (layer "F.Cu") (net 4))
 (segment (start 98.3 106.3) (end 99 107) (width 0.25) (layer "F.Cu") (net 4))
 (segment (start 99 107) (end 102.75 107) (width 0.25) (layer "F.Cu") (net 4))
 (segment (start 98.3 106) (end 98.3 106.3) (width 0.25) (layer "F.Cu") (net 4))
 (segment (start 102.9125 106.8375) (end 102.9125 106) (width 0.25) (layer "F.Cu") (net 4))
 (segment (start 96.7 106) (end 96 106) (width 0.25) (layer "F.Cu") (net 1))
 (segment (start 96 106) (end 95.75 106.25) (width 0.25) (layer "F.Cu") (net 1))
 (segment (start 95.75 106.25) (end 95.75 108.75) (width 0.25) (layer "F.Cu") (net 1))
 (via (at 95.75 108.75) (size 0.8) (drill 0.4) (layers "F.Cu" "B.Cu") (free yes) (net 1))
 (segment (start 108.5 97.195) (end 104.805 97.195) (width 0.25) (layer "F.Cu") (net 3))
 (segment (start 103 99) (end 103 103) (width 0.25) (layer "F.Cu") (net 3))
 (segment (start 104.805 97.195) (end 103 99) (width 0.25) (layer "F.Cu") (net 3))
 (segment (start 101.0875 104.9125) (end 101.0875 106) (width 0.25) (layer "F.Cu") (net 3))
 (segment (start 103 103) (end 101.0875 104.9125) (width 0.25) (layer "F.Cu") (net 3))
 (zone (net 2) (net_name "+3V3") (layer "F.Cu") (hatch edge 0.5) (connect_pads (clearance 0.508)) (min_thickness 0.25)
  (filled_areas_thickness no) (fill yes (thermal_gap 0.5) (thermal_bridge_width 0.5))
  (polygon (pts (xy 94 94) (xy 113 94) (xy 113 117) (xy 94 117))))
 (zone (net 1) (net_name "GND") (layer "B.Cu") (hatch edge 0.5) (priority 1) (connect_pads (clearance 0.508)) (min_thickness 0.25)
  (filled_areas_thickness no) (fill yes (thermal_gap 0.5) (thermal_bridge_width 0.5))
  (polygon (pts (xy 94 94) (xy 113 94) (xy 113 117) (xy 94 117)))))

